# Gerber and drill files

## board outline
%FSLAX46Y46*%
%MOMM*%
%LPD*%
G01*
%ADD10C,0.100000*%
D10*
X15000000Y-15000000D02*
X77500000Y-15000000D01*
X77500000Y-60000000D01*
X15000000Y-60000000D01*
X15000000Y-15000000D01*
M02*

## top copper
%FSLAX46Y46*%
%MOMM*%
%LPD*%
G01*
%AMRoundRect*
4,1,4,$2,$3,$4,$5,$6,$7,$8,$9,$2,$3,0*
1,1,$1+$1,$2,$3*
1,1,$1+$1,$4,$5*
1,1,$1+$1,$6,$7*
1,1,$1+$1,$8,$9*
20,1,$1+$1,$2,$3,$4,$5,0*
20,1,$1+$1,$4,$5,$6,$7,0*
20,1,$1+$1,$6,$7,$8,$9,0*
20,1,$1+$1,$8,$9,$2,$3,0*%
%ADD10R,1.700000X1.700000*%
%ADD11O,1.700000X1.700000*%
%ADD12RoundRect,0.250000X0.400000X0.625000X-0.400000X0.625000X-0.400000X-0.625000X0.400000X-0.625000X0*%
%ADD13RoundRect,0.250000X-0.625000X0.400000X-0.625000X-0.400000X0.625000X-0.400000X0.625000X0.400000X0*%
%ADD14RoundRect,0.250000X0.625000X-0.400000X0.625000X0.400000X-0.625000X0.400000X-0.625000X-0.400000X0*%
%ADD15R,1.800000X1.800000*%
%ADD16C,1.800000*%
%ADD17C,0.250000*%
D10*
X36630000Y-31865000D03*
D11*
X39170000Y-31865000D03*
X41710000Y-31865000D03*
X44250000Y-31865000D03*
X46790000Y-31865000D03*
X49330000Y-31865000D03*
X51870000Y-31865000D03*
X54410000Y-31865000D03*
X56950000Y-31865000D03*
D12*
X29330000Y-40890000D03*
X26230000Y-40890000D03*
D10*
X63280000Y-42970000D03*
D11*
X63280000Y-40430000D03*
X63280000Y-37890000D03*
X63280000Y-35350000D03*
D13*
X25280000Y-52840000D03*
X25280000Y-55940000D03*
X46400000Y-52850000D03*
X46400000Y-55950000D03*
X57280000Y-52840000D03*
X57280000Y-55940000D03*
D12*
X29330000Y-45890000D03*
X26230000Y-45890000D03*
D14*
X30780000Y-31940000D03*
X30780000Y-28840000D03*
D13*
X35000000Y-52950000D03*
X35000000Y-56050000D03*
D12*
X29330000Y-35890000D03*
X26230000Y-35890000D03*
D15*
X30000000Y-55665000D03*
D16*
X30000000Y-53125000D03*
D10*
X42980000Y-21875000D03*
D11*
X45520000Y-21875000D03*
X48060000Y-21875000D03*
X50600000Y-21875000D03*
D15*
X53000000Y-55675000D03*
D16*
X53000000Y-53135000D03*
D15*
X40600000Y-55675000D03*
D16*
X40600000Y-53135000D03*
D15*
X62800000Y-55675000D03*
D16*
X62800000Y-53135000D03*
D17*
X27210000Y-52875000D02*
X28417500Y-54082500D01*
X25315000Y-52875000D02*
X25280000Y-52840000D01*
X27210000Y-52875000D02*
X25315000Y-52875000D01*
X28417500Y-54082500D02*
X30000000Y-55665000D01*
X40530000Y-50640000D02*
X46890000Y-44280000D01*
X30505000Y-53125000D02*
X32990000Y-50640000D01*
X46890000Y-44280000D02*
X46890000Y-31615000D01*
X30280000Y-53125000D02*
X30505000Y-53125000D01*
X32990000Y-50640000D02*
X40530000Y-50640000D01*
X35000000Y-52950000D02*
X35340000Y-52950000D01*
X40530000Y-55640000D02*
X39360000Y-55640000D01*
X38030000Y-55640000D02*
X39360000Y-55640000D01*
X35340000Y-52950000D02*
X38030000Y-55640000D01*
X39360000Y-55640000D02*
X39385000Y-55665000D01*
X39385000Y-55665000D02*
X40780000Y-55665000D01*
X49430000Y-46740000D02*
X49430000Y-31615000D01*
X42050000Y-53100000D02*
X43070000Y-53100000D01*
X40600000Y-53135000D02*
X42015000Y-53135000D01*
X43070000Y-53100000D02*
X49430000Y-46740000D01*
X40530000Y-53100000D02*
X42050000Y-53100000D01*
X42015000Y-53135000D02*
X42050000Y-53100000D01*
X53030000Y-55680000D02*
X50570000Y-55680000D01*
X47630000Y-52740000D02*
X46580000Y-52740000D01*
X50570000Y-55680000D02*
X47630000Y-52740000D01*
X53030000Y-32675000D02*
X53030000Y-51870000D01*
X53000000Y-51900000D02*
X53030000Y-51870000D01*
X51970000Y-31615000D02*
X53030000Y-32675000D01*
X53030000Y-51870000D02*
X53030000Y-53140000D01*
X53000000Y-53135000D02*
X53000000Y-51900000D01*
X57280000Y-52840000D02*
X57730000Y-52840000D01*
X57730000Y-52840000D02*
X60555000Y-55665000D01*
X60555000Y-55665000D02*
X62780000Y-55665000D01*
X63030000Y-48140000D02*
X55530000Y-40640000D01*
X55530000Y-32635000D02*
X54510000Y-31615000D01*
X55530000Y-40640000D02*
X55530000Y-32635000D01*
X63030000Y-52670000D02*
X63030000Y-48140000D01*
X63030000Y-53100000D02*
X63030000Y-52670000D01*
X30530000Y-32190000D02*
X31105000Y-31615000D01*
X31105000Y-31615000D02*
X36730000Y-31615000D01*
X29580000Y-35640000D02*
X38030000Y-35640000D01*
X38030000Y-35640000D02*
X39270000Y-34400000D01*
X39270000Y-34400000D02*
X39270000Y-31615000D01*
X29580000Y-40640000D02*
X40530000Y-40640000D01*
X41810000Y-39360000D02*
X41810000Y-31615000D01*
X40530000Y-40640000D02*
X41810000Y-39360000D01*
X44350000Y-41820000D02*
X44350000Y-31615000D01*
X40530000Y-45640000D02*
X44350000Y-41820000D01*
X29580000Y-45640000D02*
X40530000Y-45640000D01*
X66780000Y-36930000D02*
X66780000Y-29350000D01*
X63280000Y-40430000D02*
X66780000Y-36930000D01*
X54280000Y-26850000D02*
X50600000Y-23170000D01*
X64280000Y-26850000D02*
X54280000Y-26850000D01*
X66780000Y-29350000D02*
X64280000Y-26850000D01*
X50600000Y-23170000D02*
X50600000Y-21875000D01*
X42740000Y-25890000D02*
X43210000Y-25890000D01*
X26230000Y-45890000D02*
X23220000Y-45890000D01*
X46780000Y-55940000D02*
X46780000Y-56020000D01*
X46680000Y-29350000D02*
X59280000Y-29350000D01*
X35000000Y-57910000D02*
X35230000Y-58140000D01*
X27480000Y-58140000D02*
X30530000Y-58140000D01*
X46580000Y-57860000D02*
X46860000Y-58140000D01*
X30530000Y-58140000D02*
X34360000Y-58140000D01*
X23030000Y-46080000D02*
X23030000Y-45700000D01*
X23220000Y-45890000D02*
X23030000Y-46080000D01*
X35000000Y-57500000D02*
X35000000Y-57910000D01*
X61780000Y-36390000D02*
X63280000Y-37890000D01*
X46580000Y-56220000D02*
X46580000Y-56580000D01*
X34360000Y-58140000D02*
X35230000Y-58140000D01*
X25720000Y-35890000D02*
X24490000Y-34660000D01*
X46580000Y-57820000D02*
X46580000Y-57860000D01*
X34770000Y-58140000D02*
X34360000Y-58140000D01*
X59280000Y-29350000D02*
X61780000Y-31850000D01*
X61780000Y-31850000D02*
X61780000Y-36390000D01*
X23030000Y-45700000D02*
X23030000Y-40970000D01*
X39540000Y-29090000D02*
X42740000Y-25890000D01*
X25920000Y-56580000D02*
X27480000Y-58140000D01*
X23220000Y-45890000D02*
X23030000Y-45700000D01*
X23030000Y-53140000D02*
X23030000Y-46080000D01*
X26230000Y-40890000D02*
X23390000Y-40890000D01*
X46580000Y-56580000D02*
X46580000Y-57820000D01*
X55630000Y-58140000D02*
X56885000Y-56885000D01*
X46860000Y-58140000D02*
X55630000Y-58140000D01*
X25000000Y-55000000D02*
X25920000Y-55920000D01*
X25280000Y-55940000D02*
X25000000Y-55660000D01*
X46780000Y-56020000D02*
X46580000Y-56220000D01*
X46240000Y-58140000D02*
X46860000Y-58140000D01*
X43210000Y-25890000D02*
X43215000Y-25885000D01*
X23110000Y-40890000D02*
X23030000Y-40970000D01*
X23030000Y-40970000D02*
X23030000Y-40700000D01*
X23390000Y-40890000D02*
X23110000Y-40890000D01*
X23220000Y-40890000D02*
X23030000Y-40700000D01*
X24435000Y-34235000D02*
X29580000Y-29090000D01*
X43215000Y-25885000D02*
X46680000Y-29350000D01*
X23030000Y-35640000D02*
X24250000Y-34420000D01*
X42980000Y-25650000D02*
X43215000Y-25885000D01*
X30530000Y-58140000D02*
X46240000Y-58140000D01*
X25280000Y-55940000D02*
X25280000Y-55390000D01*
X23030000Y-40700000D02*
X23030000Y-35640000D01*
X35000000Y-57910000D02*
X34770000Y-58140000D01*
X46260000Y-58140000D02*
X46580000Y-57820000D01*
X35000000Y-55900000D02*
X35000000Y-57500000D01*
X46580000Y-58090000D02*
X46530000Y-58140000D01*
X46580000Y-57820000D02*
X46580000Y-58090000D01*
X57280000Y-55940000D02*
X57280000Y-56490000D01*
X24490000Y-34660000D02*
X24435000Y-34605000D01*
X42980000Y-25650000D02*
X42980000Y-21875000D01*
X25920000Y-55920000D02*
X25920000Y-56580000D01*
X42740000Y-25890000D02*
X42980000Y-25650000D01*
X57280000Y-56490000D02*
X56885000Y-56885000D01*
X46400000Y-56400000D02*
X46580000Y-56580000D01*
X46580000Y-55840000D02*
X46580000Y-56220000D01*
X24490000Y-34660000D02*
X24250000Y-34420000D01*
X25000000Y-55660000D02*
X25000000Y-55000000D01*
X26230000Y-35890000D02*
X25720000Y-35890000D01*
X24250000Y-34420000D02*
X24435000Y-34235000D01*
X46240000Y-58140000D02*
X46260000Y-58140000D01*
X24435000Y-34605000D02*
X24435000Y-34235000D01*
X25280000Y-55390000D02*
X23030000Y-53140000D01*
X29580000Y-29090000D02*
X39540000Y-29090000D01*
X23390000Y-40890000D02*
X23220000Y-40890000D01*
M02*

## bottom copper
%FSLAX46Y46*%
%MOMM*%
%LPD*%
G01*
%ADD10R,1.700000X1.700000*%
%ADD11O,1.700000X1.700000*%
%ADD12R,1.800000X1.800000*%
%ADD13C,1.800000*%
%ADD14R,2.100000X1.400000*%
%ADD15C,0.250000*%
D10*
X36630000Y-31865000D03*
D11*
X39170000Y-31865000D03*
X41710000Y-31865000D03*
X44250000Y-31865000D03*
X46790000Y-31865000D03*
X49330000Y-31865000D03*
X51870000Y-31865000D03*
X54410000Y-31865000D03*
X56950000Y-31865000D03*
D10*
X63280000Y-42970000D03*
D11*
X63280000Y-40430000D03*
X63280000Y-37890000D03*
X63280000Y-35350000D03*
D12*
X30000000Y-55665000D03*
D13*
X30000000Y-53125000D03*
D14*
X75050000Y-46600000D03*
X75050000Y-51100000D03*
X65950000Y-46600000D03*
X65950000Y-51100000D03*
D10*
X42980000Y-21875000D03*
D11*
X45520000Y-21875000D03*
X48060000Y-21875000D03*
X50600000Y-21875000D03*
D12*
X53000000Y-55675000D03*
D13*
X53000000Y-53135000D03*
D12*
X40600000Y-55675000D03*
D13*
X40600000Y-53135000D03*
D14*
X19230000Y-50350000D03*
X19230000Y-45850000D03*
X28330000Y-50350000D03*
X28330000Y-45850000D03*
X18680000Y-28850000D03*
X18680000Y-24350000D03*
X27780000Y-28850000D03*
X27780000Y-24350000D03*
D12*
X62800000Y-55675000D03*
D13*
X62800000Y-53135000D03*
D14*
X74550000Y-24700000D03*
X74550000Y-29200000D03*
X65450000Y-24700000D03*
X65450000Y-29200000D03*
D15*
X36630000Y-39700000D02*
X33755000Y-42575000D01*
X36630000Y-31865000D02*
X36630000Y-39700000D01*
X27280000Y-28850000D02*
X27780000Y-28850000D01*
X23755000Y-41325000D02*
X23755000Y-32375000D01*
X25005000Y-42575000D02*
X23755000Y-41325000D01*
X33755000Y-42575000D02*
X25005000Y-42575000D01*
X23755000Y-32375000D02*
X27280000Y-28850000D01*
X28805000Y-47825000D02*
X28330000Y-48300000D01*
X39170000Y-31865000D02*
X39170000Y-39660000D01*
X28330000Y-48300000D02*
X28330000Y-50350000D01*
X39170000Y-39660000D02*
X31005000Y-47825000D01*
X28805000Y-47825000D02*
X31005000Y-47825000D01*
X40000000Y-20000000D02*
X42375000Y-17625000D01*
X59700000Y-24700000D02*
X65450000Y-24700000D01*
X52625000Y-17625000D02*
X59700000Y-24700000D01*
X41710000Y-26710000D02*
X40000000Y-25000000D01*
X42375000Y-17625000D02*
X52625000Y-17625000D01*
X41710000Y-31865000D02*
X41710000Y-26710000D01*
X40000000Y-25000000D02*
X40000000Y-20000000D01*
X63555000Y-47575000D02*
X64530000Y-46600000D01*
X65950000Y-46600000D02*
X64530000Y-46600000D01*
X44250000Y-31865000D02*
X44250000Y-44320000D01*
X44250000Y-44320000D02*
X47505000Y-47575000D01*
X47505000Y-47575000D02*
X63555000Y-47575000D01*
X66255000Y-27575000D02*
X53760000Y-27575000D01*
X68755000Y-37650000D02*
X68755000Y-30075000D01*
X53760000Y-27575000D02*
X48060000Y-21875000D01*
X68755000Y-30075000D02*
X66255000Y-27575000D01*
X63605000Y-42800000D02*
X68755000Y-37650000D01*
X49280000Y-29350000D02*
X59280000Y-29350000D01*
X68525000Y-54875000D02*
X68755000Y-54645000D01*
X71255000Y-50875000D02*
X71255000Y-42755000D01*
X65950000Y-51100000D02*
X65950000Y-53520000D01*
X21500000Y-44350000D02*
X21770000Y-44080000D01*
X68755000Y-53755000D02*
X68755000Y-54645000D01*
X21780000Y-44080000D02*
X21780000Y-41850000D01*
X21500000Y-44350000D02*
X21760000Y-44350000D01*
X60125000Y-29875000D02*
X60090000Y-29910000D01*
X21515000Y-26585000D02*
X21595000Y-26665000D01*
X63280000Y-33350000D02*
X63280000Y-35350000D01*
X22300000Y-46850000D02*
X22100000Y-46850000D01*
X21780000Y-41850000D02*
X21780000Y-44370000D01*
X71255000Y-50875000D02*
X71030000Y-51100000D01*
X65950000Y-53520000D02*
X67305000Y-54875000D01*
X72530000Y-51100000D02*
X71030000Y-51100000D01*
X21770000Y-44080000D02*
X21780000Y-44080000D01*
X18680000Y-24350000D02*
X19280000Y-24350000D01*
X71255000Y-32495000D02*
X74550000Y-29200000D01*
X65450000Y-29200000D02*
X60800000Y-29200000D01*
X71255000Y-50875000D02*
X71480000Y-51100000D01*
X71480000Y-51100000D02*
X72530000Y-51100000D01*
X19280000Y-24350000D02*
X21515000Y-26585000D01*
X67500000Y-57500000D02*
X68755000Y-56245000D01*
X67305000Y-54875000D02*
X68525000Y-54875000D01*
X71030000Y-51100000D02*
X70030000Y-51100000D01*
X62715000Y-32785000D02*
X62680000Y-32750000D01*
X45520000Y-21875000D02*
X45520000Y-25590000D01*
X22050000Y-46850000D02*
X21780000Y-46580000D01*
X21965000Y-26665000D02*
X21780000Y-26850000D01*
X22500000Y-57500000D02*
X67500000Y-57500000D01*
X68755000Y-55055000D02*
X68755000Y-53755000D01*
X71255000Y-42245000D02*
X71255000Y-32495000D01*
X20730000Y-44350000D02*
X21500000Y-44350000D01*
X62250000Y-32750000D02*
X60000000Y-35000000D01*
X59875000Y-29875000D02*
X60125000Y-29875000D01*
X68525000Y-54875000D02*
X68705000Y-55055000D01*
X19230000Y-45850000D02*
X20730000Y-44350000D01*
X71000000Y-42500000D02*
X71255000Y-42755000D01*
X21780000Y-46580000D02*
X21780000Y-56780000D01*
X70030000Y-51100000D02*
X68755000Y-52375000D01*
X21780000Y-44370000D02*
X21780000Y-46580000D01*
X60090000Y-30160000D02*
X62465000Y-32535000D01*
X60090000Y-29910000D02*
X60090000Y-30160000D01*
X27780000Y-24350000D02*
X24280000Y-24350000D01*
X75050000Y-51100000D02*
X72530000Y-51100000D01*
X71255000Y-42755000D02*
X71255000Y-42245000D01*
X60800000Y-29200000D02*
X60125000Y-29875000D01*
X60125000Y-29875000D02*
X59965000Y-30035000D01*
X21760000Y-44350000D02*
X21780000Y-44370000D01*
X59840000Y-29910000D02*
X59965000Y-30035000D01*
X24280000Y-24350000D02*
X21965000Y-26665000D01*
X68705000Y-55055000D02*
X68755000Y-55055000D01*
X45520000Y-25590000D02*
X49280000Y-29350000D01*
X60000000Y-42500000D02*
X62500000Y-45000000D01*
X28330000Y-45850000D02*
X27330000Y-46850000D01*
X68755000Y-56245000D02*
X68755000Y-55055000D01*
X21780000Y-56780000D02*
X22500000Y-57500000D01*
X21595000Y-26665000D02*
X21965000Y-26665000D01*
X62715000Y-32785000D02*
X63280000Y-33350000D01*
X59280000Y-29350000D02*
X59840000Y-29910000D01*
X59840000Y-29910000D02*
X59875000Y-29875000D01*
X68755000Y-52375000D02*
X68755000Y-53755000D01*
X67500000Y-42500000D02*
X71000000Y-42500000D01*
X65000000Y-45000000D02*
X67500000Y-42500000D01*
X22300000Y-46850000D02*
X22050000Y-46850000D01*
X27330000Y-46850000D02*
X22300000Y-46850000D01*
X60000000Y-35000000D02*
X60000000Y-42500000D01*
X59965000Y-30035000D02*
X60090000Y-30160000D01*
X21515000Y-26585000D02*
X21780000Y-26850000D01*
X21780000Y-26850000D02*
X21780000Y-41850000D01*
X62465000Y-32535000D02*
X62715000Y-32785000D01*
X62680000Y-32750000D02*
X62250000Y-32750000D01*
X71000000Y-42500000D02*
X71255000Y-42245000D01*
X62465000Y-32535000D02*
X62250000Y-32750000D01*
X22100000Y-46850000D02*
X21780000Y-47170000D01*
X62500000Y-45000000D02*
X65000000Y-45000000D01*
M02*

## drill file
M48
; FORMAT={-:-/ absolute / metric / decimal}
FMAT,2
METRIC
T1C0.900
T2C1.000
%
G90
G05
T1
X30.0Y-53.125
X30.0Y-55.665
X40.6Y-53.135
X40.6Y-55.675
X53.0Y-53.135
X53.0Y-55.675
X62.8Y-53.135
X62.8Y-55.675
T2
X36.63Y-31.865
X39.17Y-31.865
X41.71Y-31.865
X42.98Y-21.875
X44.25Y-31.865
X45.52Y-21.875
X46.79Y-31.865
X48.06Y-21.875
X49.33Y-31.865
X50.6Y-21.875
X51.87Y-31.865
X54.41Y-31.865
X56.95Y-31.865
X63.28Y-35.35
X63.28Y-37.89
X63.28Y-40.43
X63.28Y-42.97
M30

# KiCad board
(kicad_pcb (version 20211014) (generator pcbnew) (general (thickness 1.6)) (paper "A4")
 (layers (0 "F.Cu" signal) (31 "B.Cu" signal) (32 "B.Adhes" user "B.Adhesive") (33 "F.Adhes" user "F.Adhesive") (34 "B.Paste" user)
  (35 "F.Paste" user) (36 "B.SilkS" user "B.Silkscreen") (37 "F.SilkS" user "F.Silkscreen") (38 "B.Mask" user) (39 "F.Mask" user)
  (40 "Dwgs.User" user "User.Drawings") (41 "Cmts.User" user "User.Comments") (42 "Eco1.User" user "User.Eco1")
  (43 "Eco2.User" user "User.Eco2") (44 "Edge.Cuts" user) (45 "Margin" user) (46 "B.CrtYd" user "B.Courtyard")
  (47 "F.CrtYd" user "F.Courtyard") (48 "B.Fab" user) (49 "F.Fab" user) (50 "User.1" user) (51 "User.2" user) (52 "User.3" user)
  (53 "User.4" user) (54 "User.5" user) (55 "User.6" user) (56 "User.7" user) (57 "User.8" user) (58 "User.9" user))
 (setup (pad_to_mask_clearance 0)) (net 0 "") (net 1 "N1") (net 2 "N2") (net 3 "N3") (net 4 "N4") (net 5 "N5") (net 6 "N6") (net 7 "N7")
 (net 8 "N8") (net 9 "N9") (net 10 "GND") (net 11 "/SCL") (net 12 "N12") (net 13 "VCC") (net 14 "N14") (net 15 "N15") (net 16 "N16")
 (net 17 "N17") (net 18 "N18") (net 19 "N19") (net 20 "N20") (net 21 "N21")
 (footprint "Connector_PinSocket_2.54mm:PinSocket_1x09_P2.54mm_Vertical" (layer "F.Cu") (at 36.63 31.865 90)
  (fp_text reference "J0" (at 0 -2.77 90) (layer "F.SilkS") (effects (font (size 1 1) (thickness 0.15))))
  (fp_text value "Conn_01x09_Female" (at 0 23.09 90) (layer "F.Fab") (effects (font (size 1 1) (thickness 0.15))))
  (pad "1" thru_hole rect (at 0 0 90) (size 1.7 1.7) (drill 1) (layers *.Cu *.Mask) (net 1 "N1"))
  (pad "2" thru_hole oval (at 0 2.54 90) (size 1.7 1.7) (drill 1) (layers *.Cu *.Mask) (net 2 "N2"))
  (pad "3" thru_hole oval (at 0 5.08 90) (size 1.7 1.7) (drill 1) (layers *.Cu *.Mask) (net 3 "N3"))
  (pad "4" thru_hole oval (at 0 7.62 90) (size 1.7 1.7) (drill 1) (layers *.Cu *.Mask) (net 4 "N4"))
  (pad "5" thru_hole oval (at 0 10.16 90) (size 1.7 1.7) (drill 1) (layers *.Cu *.Mask) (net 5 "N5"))
  (pad "6" thru_hole oval (at 0 12.7 90) (size 1.7 1.7) (drill 1) (layers *.Cu *.Mask) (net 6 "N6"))
  (pad "7" thru_hole oval (at 0 15.24 90) (size 1.7 1.7) (drill 1) (layers *.Cu *.Mask) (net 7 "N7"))
  (pad "8" thru_hole oval (at 0 17.78 90) (size 1.7 1.7) (drill 1) (layers *.Cu *.Mask) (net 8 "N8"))
  (pad "9" thru_hole oval (at 0 20.32 90) (size 1.7 1.7) (drill 1) (layers *.Cu *.Mask) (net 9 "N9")))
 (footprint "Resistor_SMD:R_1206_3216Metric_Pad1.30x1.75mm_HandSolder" (layer "F.Cu") (at 27.78 40.89 180)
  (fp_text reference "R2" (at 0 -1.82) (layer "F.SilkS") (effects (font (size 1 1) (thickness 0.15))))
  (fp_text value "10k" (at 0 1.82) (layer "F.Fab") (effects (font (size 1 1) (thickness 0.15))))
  (pad "1" smd roundrect (at -1.55 0 180) (size 1.3 1.75) (layers "F.Cu" "F.Paste" "F.Mask") (roundrect_rratio 0.192308) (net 3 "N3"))
  (pad "2" smd roundrect (at 1.55 0 180) (size 1.3 1.75) (layers "F.Cu" "F.Paste" "F.Mask") (roundrect_rratio 0.192308) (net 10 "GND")))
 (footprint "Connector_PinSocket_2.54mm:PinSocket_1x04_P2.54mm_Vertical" (layer "F.Cu") (at 63.28 42.97 180)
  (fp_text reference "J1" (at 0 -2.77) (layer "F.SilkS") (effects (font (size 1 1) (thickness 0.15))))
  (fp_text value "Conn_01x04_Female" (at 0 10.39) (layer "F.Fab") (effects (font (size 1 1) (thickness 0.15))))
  (pad "1" thru_hole rect (at 0 0 180) (size 1.7 1.7) (drill 1) (layers *.Cu *.Mask) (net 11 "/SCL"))
  (pad "2" thru_hole oval (at 0 2.54 180) (size 1.7 1.7) (drill 1) (layers *.Cu *.Mask) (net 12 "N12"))
  (pad "3" thru_hole oval (at 0 5.08 180) (size 1.7 1.7) (drill 1) (layers *.Cu *.Mask) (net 10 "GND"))
  (pad "4" thru_hole oval (at 0 7.62 180) (size 1.7 1.7) (drill 1) (layers *.Cu *.Mask) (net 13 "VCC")))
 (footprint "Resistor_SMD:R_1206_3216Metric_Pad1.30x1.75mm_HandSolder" (layer "F.Cu") (at 25.28 54.39 -90)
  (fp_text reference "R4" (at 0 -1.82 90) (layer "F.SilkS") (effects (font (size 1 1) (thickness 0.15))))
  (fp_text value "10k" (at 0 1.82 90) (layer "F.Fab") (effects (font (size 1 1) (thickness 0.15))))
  (pad "1" smd roundrect (at -1.55 0 270) (size 1.3 1.75) (layers "F.Cu" "F.Paste" "F.Mask") (roundrect_rratio 0.192308) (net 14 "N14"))
  (pad "2" smd roundrect (at 1.55 0 270) (size 1.3 1.75) (layers "F.Cu" "F.Paste" "F.Mask") (roundrect_rratio 0.192308) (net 10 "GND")))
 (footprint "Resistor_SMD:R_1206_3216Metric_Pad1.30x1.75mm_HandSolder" (layer "F.Cu") (at 46.4 54.4 -90)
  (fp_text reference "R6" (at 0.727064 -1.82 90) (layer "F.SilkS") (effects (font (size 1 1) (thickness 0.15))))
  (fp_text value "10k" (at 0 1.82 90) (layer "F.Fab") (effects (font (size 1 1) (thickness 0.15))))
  (pad "1" smd roundrect (at -1.55 0 270) (size 1.3 1.75) (layers "F.Cu" "F.Paste" "F.Mask") (roundrect_rratio 0.192308) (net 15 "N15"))
  (pad "2" smd roundrect (at 1.55 0 270) (size 1.3 1.75) (layers "F.Cu" "F.Paste" "F.Mask") (roundrect_rratio 0.192308) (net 10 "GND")))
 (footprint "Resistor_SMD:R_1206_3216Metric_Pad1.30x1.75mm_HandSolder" (layer "F.Cu") (at 57.28 54.39 -90)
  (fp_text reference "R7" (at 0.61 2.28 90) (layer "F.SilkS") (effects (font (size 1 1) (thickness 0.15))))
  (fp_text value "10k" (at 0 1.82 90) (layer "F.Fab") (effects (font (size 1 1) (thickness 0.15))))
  (pad "1" smd roundrect (at -1.55 0 270) (size 1.3 1.75) (layers "F.Cu" "F.Paste" "F.Mask") (roundrect_rratio 0.192308) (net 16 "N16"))
  (pad "2" smd roundrect (at 1.55 0 270) (size 1.3 1.75) (layers "F.Cu" "F.Paste" "F.Mask") (roundrect_rratio 0.192308) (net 10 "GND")))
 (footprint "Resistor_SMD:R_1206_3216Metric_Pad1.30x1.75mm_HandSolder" (layer "F.Cu") (at 27.78 45.89 180)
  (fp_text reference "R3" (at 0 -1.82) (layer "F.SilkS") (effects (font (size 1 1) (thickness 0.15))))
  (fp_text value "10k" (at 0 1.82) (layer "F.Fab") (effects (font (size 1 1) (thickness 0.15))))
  (pad "1" smd roundrect (at -1.55 0 180) (size 1.3 1.75) (layers "F.Cu" "F.Paste" "F.Mask") (roundrect_rratio 0.192308) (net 4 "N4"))
  (pad "2" smd roundrect (at 1.55 0 180) (size 1.3 1.75) (layers "F.Cu" "F.Paste" "F.Mask") (roundrect_rratio 0.192308) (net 10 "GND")))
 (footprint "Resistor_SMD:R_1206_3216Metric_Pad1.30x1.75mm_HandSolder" (layer "F.Cu") (at 30.78 30.39 90)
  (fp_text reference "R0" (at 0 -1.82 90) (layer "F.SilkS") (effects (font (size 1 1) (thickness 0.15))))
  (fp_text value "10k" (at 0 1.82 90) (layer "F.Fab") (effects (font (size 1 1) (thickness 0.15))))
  (pad "1" smd roundrect (at -1.55 0 90) (size 1.3 1.75) (layers "F.Cu" "F.Paste" "F.Mask") (roundrect_rratio 0.192308) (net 1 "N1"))
  (pad "2" smd roundrect (at 1.55 0 90) (size 1.3 1.75) (layers "F.Cu" "F.Paste" "F.Mask") (roundrect_rratio 0.192308) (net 10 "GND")))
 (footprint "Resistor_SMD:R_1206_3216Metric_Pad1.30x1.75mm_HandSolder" (layer "F.Cu") (at 35 54.5 -90)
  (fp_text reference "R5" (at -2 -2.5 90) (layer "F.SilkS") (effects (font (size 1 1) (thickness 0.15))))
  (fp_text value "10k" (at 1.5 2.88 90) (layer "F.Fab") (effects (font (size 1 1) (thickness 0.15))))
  (pad "1" smd roundrect (at -1.55 0 270) (size 1.3 1.75) (layers "F.Cu" "F.Paste" "F.Mask") (roundrect_rratio 0.192308) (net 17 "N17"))
  (pad "2" smd roundrect (at 1.55 0 270) (size 1.3 1.75) (layers "F.Cu" "F.Paste" "F.Mask") (roundrect_rratio 0.192308) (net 10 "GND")))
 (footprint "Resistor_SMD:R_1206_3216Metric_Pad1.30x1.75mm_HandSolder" (layer "F.Cu") (at 27.78 35.89 180)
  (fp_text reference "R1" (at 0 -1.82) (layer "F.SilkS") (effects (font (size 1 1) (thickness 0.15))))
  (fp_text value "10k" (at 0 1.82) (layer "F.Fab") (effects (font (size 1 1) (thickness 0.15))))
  (pad "1" smd roundrect (at -1.55 0 180) (size 1.3 1.75) (layers "F.Cu" "F.Paste" "F.Mask") (roundrect_rratio 0.192308) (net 2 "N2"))
  (pad "2" smd roundrect (at 1.55 0 180) (size 1.3 1.75) (layers "F.Cu" "F.Paste" "F.Mask") (roundrect_rratio 0.192308) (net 10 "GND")))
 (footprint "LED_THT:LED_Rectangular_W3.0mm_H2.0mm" (layer "B.Cu") (at 30 55.665 90)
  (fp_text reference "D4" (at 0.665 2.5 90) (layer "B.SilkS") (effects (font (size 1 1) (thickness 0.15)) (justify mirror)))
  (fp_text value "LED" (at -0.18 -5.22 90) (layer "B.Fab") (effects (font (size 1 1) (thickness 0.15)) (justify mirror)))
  (pad "1" thru_hole rect (at 0 0 90) (size 1.8 1.8) (drill 0.9) (layers *.Cu *.Mask) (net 14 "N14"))
  (pad "2" thru_hole circle (at 2.54 0 90) (size 1.8 1.8) (drill 0.9) (layers *.Cu *.Mask) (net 5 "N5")))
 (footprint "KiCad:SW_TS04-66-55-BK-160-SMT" (layer "B.Cu") (at 70.5 48.85 180)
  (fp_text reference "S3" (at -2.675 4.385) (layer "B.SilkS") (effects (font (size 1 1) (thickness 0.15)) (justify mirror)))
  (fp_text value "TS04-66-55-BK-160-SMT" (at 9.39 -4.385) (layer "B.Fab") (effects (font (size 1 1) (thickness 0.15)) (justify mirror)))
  (pad "1" smd rect locked (at -4.55 2.25 180) (size 2.1 1.4) (layers "B.Cu" "B.Paste" "B.Mask") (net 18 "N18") (solder_mask_margin 0.102))
  (pad "2" smd rect locked (at -4.55 -2.25 180) (size 2.1 1.4) (layers "B.Cu" "B.Paste" "B.Mask") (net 13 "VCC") (solder_mask_margin 0.102))
  (pad "3" smd rect locked (at 4.55 2.25 180) (size 2.1 1.4) (layers "B.Cu" "B.Paste" "B.Mask") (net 4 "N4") (solder_mask_margin 0.102))
  (pad "4" smd rect locked (at 4.55 -2.25 180) (size 2.1 1.4) (layers "B.Cu" "B.Paste" "B.Mask") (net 13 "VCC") (solder_mask_margin 0.102)))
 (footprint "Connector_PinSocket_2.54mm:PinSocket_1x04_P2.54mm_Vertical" (layer "B.Cu") (at 42.98 21.875 -90)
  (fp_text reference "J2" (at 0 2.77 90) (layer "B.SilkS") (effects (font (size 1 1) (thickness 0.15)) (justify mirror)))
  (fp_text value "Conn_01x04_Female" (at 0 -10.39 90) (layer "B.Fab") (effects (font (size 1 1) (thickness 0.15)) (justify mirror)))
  (pad "1" thru_hole rect (at 0 0 270) (size 1.7 1.7) (drill 1) (layers *.Cu *.Mask) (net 10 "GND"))
  (pad "2" thru_hole oval (at 0 -2.54 270) (size 1.7 1.7) (drill 1) (layers *.Cu *.Mask) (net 13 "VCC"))
  (pad "3" thru_hole oval (at 0 -5.08 270) (size 1.7 1.7) (drill 1) (layers *.Cu *.Mask) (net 11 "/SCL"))
  (pad "4" thru_hole oval (at 0 -7.62 270) (size 1.7 1.7) (drill 1) (layers *.Cu *.Mask) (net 12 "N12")))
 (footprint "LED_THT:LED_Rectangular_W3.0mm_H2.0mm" (layer "B.Cu") (at 53 55.675 90)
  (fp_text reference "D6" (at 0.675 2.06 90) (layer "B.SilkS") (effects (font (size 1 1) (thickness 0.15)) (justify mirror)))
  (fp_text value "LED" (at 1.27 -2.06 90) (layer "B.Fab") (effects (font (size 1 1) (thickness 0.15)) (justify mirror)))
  (pad "1" thru_hole rect (at 0 0 90) (size 1.8 1.8) (drill 0.9) (layers *.Cu *.Mask) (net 15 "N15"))
  (pad "2" thru_hole circle (at 2.54 0 90) (size 1.8 1.8) (drill 0.9) (layers *.Cu *.Mask) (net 7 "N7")))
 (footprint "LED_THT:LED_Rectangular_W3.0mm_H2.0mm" (layer "B.Cu") (at 40.6 55.675 90)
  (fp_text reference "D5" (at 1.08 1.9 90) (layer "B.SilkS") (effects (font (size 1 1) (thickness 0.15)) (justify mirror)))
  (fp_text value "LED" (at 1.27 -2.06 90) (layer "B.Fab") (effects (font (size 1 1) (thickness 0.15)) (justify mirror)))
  (pad "1" thru_hole rect (at 0 0 90) (size 1.8 1.8) (drill 0.9) (layers *.Cu *.Mask) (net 17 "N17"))
  (pad "2" thru_hole circle (at 2.54 0 90) (size 1.8 1.8) (drill 0.9) (layers *.Cu *.Mask) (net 6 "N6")))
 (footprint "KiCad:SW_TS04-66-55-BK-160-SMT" (layer "B.Cu") (at 23.78 48.1)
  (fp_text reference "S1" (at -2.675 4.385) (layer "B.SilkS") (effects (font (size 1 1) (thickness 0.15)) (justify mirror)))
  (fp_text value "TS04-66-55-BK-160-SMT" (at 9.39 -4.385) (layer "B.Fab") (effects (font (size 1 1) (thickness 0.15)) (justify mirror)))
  (pad "1" smd rect locked (at -4.55 2.25) (size 2.1 1.4) (layers "B.Cu" "B.Paste" "B.Mask") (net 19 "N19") (solder_mask_margin 0.102))
  (pad "2" smd rect locked (at -4.55 -2.25) (size 2.1 1.4) (layers "B.Cu" "B.Paste" "B.Mask") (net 13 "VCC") (solder_mask_margin 0.102))
  (pad "3" smd rect locked (at 4.55 2.25) (size 2.1 1.4) (layers "B.Cu" "B.Paste" "B.Mask") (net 2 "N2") (solder_mask_margin 0.102))
  (pad "4" smd rect locked (at 4.55 -2.25) (size 2.1 1.4) (layers "B.Cu" "B.Paste" "B.Mask") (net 13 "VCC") (solder_mask_margin 0.102)))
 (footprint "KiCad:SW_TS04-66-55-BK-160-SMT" (layer "B.Cu") (at 23.23 26.6)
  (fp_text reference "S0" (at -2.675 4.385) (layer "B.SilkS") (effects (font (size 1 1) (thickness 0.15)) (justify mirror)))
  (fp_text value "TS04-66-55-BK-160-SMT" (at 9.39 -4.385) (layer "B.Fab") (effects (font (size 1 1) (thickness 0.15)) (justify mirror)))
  (pad "1" smd rect locked (at -4.55 2.25) (size 2.1 1.4) (layers "B.Cu" "B.Paste" "B.Mask") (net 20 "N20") (solder_mask_margin 0.102))
  (pad "2" smd rect locked (at -4.55 -2.25) (size 2.1 1.4) (layers "B.Cu" "B.Paste" "B.Mask") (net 13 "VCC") (solder_mask_margin 0.102))
  (pad "3" smd rect locked (at 4.55 2.25) (size 2.1 1.4) (layers "B.Cu" "B.Paste" "B.Mask") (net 1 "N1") (solder_mask_margin 0.102))
  (pad "4" smd rect locked (at 4.55 -2.25) (size 2.1 1.4) (layers "B.Cu" "B.Paste" "B.Mask") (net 13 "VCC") (solder_mask_margin 0.102)))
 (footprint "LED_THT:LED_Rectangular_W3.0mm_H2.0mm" (layer "B.Cu") (at 62.8 55.675 90)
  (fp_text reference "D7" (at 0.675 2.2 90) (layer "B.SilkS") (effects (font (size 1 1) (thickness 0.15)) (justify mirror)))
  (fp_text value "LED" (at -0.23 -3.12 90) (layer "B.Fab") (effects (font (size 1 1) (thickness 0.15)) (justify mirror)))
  (pad "1" thru_hole rect (at 0 0 90) (size 1.8 1.8) (drill 0.9) (layers *.Cu *.Mask) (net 16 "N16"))
  (pad "2" thru_hole circle (at 2.54 0 90) (size 1.8 1.8) (drill 0.9) (layers *.Cu *.Mask) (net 8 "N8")))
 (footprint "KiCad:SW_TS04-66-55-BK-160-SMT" (layer "B.Cu") (at 70 26.95 180)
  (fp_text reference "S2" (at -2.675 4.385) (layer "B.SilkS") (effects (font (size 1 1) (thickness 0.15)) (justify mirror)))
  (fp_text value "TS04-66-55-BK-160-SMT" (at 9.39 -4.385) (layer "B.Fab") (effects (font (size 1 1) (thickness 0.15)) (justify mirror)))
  (pad "1" smd rect locked (at -4.55 2.25 180) (size 2.1 1.4) (layers "B.Cu" "B.Paste" "B.Mask") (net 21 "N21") (solder_mask_margin 0.102))
  (pad "2" smd rect locked (at -4.55 -2.25 180) (size 2.1 1.4) (layers "B.Cu" "B.Paste" "B.Mask") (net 13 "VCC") (solder_mask_margin 0.102))
  (pad "3" smd rect locked (at 4.55 2.25 180) (size 2.1 1.4) (layers "B.Cu" "B.Paste" "B.Mask") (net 3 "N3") (solder_mask_margin 0.102))
  (pad "4" smd rect locked (at 4.55 -2.25 180) (size 2.1 1.4) (layers "B.Cu" "B.Paste" "B.Mask") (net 13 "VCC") (solder_mask_margin 0.102)))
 (gr_rect (start 15 15) (end 77.5 60) (layer "Edge.Cuts") (width 0.1) (fill none))
 (gr_rect (start 12.5 15) (end 12.5 15) (layer "Edge.Cuts") (width 0.1) (fill none))
 (segment (start 27.21 52.875) (end 28.4175 54.0825) (width 0.25) (layer "F.Cu") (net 14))
 (segment (start 25.315 52.875) (end 25.28 52.84) (width 0.25) (layer "F.Cu") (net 14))
 (segment (start 27.21 52.875) (end 25.315 52.875) (width 0.25) (layer "F.Cu") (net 14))
 (segment (start 28.4175 54.0825) (end 30 55.665) (width 0.25) (layer "F.Cu") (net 14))
 (segment (start 40.53 50.64) (end 46.89 44.28) (width 0.25) (layer "F.Cu") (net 5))
 (segment (start 30.505 53.125) (end 32.99 50.64) (width 0.25) (layer "F.Cu") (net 5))
 (segment (start 46.89 44.28) (end 46.89 31.615) (width 0.25) (layer "F.Cu") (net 5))
 (segment (start 30.28 53.125) (end 30.505 53.125) (width 0.25) (layer "F.Cu") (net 5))
 (segment (start 32.99 50.64) (end 40.53 50.64) (width 0.25) (layer "F.Cu") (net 5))
 (segment (start 35 52.95) (end 35.34 52.95) (width 0.25) (layer "F.Cu") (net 17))
 (segment (start 40.53 55.64) (end 39.36 55.64) (width 0.25) (layer "F.Cu") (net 17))
 (segment (start 38.03 55.64) (end 39.36 55.64) (width 0.25) (layer "F.Cu") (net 17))
 (segment (start 35.34 52.95) (end 38.03 55.64) (width 0.25) (layer "F.Cu") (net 17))
 (segment (start 39.36 55.64) (end 39.385 55.665) (width 0.25) (layer "F.Cu") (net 17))
 (segment (start 39.385 55.665) (end 40.78 55.665) (width 0.25) (layer "F.Cu") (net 17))
 (segment (start 49.43 46.74) (end 49.43 31.615) (width 0.25) (layer "F.Cu") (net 6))
 (segment (start 42.05 53.1) (end 43.07 53.1) (width 0.25) (layer "F.Cu") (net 6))
 (segment (start 40.6 53.135) (end 42.015 53.135) (width 0.25) (layer "F.Cu") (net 6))
 (segment (start 43.07 53.1) (end 49.43 46.74) (width 0.25) (layer "F.Cu") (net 6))
 (segment (start 40.53 53.1) (end 42.05 53.1) (width 0.25) (layer "F.Cu") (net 6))
 (segment (start 42.015 53.135) (end 42.05 53.1) (width 0.25) (layer "F.Cu") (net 6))
 (segment (start 53.03 55.68) (end 50.57 55.68) (width 0.25) (layer "F.Cu") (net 15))
 (segment (start 47.63 52.74) (end 46.58 52.74) (width 0.25) (layer "F.Cu") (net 15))
 (segment (start 50.57 55.68) (end 47.63 52.74) (width 0.25) (layer "F.Cu") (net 15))
 (segment (start 53.03 32.675) (end 53.03 51.87) (width 0.25) (layer "F.Cu") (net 7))
 (segment (start 53 51.9) (end 53.03 51.87) (width 0.25) (layer "F.Cu") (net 7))
 (segment (start 51.97 31.615) (end 53.03 32.675) (width 0.25) (layer "F.Cu") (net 7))
 (segment (start 53.03 51.87) (end 53.03 53.14) (width 0.25) (layer "F.Cu") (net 7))
 (segment (start 53 53.135) (end 53 51.9) (width 0.25) (layer "F.Cu") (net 7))
 (segment (start 57.28 52.84) (end 57.73 52.84) (width 0.25) (layer "F.Cu") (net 16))
 (segment (start 57.73 52.84) (end 60.555 55.665) (width 0.25) (layer "F.Cu") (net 16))
 (segment (start 60.555 55.665) (end 62.78 55.665) (width 0.25) (layer "F.Cu") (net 16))
 (segment (start 63.03 48.14) (end 55.53 40.64) (width 0.25) (layer "F.Cu") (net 8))
 (segment (start 55.53 32.635) (end 54.51 31.615) (width 0.25) (layer "F.Cu") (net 8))
 (segment (start 55.53 40.64) (end 55.53 32.635) (width 0.25) (layer "F.Cu") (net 8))
 (segment (start 63.03 52.67) (end 63.03 48.14) (width 0.25) (layer "F.Cu") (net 8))
 (segment (start 63.03 53.1) (end 63.03 52.67) (width 0.25) (layer "F.Cu") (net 8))
 (segment (start 30.53 32.19) (end 31.105 31.615) (width 0.25) (layer "F.Cu") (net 1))
 (segment (start 31.105 31.615) (end 36.73 31.615) (width 0.25) (layer "F.Cu") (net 1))
 (segment (start 36.63 39.7) (end 33.755 42.575) (width 0.25) (layer "B.Cu") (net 1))
 (segment (start 36.63 31.865) (end 36.63 39.7) (width 0.25) (layer "B.Cu") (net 1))
 (segment (start 27.28 28.85) (end 27.78 28.85) (width 0.25) (layer "B.Cu") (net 1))
 (segment (start 23.755 41.325) (end 23.755 32.375) (width 0.25) (layer "B.Cu") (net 1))
 (segment (start 25.005 42.575) (end 23.755 41.325) (width 0.25) (layer "B.Cu") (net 1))
 (segment (start 33.755 42.575) (end 25.005 42.575) (width 0.25) (layer "B.Cu") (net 1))
 (segment (start 23.755 32.375) (end 27.28 28.85) (width 0.25) (layer "B.Cu") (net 1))
 (segment (start 29.58 35.64) (end 38.03 35.64) (width 0.25) (layer "F.Cu") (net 2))
 (segment (start 38.03 35.64) (end 39.27 34.4) (width 0.25) (layer "F.Cu") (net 2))
 (segment (start 39.27 34.4) (end 39.27 31.615) (width 0.25) (layer "F.Cu") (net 2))
 (segment (start 28.805 47.825) (end 28.33 48.3) (width 0.25) (layer "B.Cu") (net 2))
 (segment (start 39.17 31.865) (end 39.17 39.66) (width 0.25) (layer "B.Cu") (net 2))
 (segment (start 28.33 48.3) (end 28.33 50.35) (width 0.25) (layer "B.Cu") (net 2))
 (segment (start 39.17 39.66) (end 31.005 47.825) (width 0.25) (layer "B.Cu") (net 2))
 (segment (start 28.805 47.825) (end 31.005 47.825) (width 0.25) (layer "B.Cu") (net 2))
 (segment (start 29.58 40.64) (end 40.53 40.64) (width 0.25) (layer "F.Cu") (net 3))
 (segment (start 41.81 39.36) (end 41.81 31.615) (width 0.25) (layer "F.Cu") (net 3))
 (segment (start 40.53 40.64) (end 41.81 39.36) (width 0.25) (layer "F.Cu") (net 3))
 (segment (start 40 20) (end 42.375 17.625) (width 0.25) (layer "B.Cu") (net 3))
 (segment (start 59.7 24.7) (end 65.45 24.7) (width 0.25) (layer "B.Cu") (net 3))
 (segment (start 52.625 17.625) (end 59.7 24.7) (width 0.25) (layer "B.Cu") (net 3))
 (segment (start 41.71 26.71) (end 40 25) (width 0.25) (layer "B.Cu") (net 3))
 (segment (start 42.375 17.625) (end 52.625 17.625) (width 0.25) (layer "B.Cu") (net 3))
 (segment (start 41.71 31.865) (end 41.71 26.71) (width 0.25) (layer "B.Cu") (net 3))
 (segment (start 40 25) (end 40 20) (width 0.25) (layer "B.Cu") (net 3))
 (segment (start 44.35 41.82) (end 44.35 31.615) (width 0.25) (layer "F.Cu") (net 4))
 (segment (start 40.53 45.64) (end 44.35 41.82) (width 0.25) (layer "F.Cu") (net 4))
 (segment (start 29.58 45.64) (end 40.53 45.64) (width 0.25) (layer "F.Cu") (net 4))
 (segment (start 63.555 47.575) (end 64.53 46.6) (width 0.25) (layer "B.Cu") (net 4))
 (segment (start 65.95 46.6) (end 64.53 46.6) (width 0.25) (layer "B.Cu") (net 4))
 (segment (start 44.25 31.865) (end 44.25 44.32) (width 0.25) (layer "B.Cu") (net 4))
 (segment (start 44.25 44.32) (end 47.505 47.575) (width 0.25) (layer "B.Cu") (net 4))
 (segment (start 47.505 47.575) (end 63.555 47.575) (width 0.25) (layer "B.Cu") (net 4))
 (segment (start 66.255 27.575) (end 53.76 27.575) (width 0.25) (layer "B.Cu") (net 11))
 (segment (start 68.755 37.65) (end 68.755 30.075) (width 0.25) (layer "B.Cu") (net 11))
 (segment (start 53.76 27.575) (end 48.06 21.875) (width 0.25) (layer "B.Cu") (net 11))
 (segment (start 68.755 30.075) (end 66.255 27.575) (width 0.25) (layer "B.Cu") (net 11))
 (segment (start 63.605 42.8) (end 68.755 37.65) (width 0.25) (layer "B.Cu") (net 11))
 (segment (start 66.78 36.93) (end 66.78 29.35) (width 0.25) (layer "F.Cu") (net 12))
 (segment (start 63.28 40.43) (end 66.78 36.93) (width 0.25) (layer "F.Cu") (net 12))
 (segment (start 54.28 26.85) (end 50.6 23.17) (width 0.25) (layer "F.Cu") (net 12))
 (segment (start 64.28 26.85) (end 54.28 26.85) (width 0.25) (layer "F.Cu") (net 12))
 (segment (start 66.78 29.35) (end 64.28 26.85) (width 0.25) (layer "F.Cu") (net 12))
 (segment (start 50.6 23.17) (end 50.6 21.875) (width 0.25) (layer "F.Cu") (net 12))
 (segment (start 42.74 25.89) (end 43.21 25.89) (width 0.25) (layer "F.Cu") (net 10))
 (segment (start 26.23 45.89) (end 23.22 45.89) (width 0.25) (layer "F.Cu") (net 10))
 (segment (start 46.78 55.94) (end 46.78 56.02) (width 0.25) (layer "F.Cu") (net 10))
 (segment (start 46.68 29.35) (end 59.28 29.35) (width 0.25) (layer "F.Cu") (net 10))
 (segment (start 35 57.91) (end 35.23 58.14) (width 0.25) (layer "F.Cu") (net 10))
 (segment (start 27.48 58.14) (end 30.53 58.14) (width 0.25) (layer "F.Cu") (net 10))
 (segment (start 46.58 57.86) (end 46.86 58.14) (width 0.25) (layer "F.Cu") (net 10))
 (segment (start 30.53 58.14) (end 34.36 58.14) (width 0.25) (layer "F.Cu") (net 10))
 (segment (start 23.03 46.08) (end 23.03 45.7) (width 0.25) (layer "F.Cu") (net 10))
 (segment (start 23.22 45.89) (end 23.03 46.08) (width 0.25) (layer "F.Cu") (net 10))
 (segment (start 35 57.5) (end 35 57.91) (width 0.25) (layer "F.Cu") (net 10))
 (segment (start 61.78 36.39) (end 63.28 37.89) (width 0.25) (layer "F.Cu") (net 10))
 (segment (start 46.58 56.22) (end 46.58 56.58) (width 0.25) (layer "F.Cu") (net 10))
 (segment (start 34.36 58.14) (end 35.23 58.14) (width 0.25) (layer "F.Cu") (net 10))
 (segment (start 25.72 35.89) (end 24.49 34.66) (width 0.25) (layer "F.Cu") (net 10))
 (segment (start 46.58 57.82) (end 46.58 57.86) (width 0.25) (layer "F.Cu") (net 10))
 (segment (start 34.77 58.14) (end 34.36 58.14) (width 0.25) (layer "F.Cu") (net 10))
 (segment (start 59.28 29.35) (end 61.78 31.85) (width 0.25) (layer "F.Cu") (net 10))
 (segment (start 61.78 31.85) (end 61.78 36.39) (width 0.25) (layer "F.Cu") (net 10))
 (segment (start 23.03 45.7) (end 23.03 40.97) (width 0.25) (layer "F.Cu") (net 10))
 (segment (start 39.54 29.09) (end 42.74 25.89) (width 0.25) (layer "F.Cu") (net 10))
 (segment (start 25.92 56.58) (end 27.48 58.14) (width 0.25) (layer "F.Cu") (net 10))
 (segment (start 23.22 45.89) (end 23.03 45.7) (width 0.25) (layer "F.Cu") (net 10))
 (segment (start 23.03 53.14) (end 23.03 46.08) (width 0.25) (layer "F.Cu") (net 10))
 (segment (start 26.23 40.89) (end 23.39 40.89) (width 0.25) (layer "F.Cu") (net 10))
 (segment (start 46.58 56.58) (end 46.58 57.82) (width 0.25) (layer "F.Cu") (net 10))
 (segment (start 55.63 58.14) (end 56.885 56.885) (width 0.25) (layer "F.Cu") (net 10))
 (segment (start 46.86 58.14) (end 55.63 58.14) (width 0.25) (layer "F.Cu") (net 10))
 (segment (start 25 55) (end 25.92 55.92) (width 0.25) (layer "F.Cu") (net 10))
 (segment (start 25.28 55.94) (end 25 55.66) (width 0.25) (layer "F.Cu") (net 10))
 (segment (start 46.78 56.02) (end 46.58 56.22) (width 0.25) (layer "F.Cu") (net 10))
 (segment (start 46.24 58.14) (end 46.86 58.14) (width 0.25) (layer "F.Cu") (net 10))
 (segment (start 43.21 25.89) (end 43.215 25.885) (width 0.25) (layer "F.Cu") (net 10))
 (segment (start 23.11 40.89) (end 23.03 40.97) (width 0.25) (layer "F.Cu") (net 10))
 (segment (start 23.03 40.97) (end 23.03 40.7) (width 0.25) (layer "F.Cu") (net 10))
 (segment (start 23.39 40.89) (end 23.11 40.89) (width 0.25) (layer "F.Cu") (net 10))
 (segment (start 23.22 40.89) (end 23.03 40.7) (width 0.25) (layer "F.Cu") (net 10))
 (segment (start 24.435 34.235) (end 29.58 29.09) (width 0.25) (layer "F.Cu") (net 10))
 (segment (start 43.215 25.885) (end 46.68 29.35) (width 0.25) (layer "F.Cu") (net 10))
 (segment (start 23.03 35.64) (end 24.25 34.42) (width 0.25) (layer "F.Cu") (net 10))
 (segment (start 42.98 25.65) (end 43.215 25.885) (width 0.25) (layer "F.Cu") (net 10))
 (segment (start 30.53 58.14) (end 46.24 58.14) (width 0.25) (layer "F.Cu") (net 10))
 (segment (start 25.28 55.94) (end 25.28 55.39) (width 0.25) (layer "F.Cu") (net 10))
 (segment (start 23.03 40.7) (end 23.03 35.64) (width 0.25) (layer "F.Cu") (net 10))
 (segment (start 35 57.91) (end 34.77 58.14) (width 0.25) (layer "F.Cu") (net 10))
 (segment (start 46.26 58.14) (end 46.58 57.82) (width 0.25) (layer "F.Cu") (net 10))
 (segment (start 35 55.9) (end 35 57.5) (width 0.25) (layer "F.Cu") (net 10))
 (segment (start 46.58 58.09) (end 46.53 58.14) (width 0.25) (layer "F.Cu") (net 10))
 (segment (start 46.58 57.82) (end 46.58 58.09) (width 0.25) (layer "F.Cu") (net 10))
 (segment (start 57.28 55.94) (end 57.28 56.49) (width 0.25) (layer "F.Cu") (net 10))
 (segment (start 24.49 34.66) (end 24.435 34.605) (width 0.25) (layer "F.Cu") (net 10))
 (segment (start 42.98 25.65) (end 42.98 21.875) (width 0.25) (layer "F.Cu") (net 10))
 (segment (start 25.92 55.92) (end 25.92 56.58) (width 0.25) (layer "F.Cu") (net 10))
 (segment (start 42.74 25.89) (end 42.98 25.65) (width 0.25) (layer "F.Cu") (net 10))
 (segment (start 57.28 56.49) (end 56.885 56.885) (width 0.25) (layer "F.Cu") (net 10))
 (segment (start 46.4 56.4) (end 46.58 56.58) (width 0.25) (layer "F.Cu") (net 10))
 (segment (start 46.58 55.84) (end 46.58 56.22) (width 0.25) (layer "F.Cu") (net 10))
 (segment (start 24.49 34.66) (end 24.25 34.42) (width 0.25) (layer "F.Cu") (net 10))
 (segment (start 25 55.66) (end 25 55) (width 0.25) (layer "F.Cu") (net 10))
 (segment (start 26.23 35.89) (end 25.72 35.89) (width 0.25) (layer "F.Cu") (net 10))
 (segment (start 24.25 34.42) (end 24.435 34.235) (width 0.25) (layer "F.Cu") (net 10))
 (segment (start 46.24 58.14) (end 46.26 58.14) (width 0.25) (layer "F.Cu") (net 10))
 (segment (start 24.435 34.605) (end 24.435 34.235) (width 0.25) (layer "F.Cu") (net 10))
 (segment (start 25.28 55.39) (end 23.03 53.14) (width 0.25) (layer "F.Cu") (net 10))
 (segment (start 29.58 29.09) (end 39.54 29.09) (width 0.25) (layer "F.Cu") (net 10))
 (segment (start 23.39 40.89) (end 23.22 40.89) (width 0.25) (layer "F.Cu") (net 10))
 (segment (start 49.28 29.35) (end 59.28 29.35) (width 0.25) (layer "B.Cu") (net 13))
 (segment (start 68.525 54.875) (end 68.755 54.645) (width 0.25) (layer "B.Cu") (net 13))
 (segment (start 71.255 50.875) (end 71.255 42.755) (width 0.25) (layer "B.Cu") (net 13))
 (segment (start 65.95 51.1) (end 65.95 53.52) (width 0.25) (layer "B.Cu") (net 13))
 (segment (start 21.5 44.35) (end 21.77 44.08) (width 0.25) (layer "B.Cu") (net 13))
 (segment (start 68.755 53.755) (end 68.755 54.645) (width 0.25) (layer "B.Cu") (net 13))
 (segment (start 21.78 44.08) (end 21.78 41.85) (width 0.25) (layer "B.Cu") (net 13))
 (segment (start 21.5 44.35) (end 21.76 44.35) (width 0.25) (layer "B.Cu") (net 13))
 (segment (start 60.125 29.875) (end 60.09 29.91) (width 0.25) (layer "B.Cu") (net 13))
 (segment (start 21.515 26.585) (end 21.595 26.665) (width 0.25) (layer "B.Cu") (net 13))
 (segment (start 63.28 33.35) (end 63.28 35.35) (width 0.25) (layer "B.Cu") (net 13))
 (segment (start 22.3 46.85) (end 22.1 46.85) (width 0.25) (layer "B.Cu") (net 13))
 (segment (start 21.78 41.85) (end 21.78 44.37) (width 0.25) (layer "B.Cu") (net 13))
 (segment (start 71.255 50.875) (end 71.03 51.1) (width 0.25) (layer "B.Cu") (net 13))
 (segment (start 65.95 53.52) (end 67.305 54.875) (width 0.25) (layer "B.Cu") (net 13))
 (segment (start 72.53 51.1) (end 71.03 51.1) (width 0.25) (layer "B.Cu") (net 13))
 (segment (start 21.77 44.08) (end 21.78 44.08) (width 0.25) (layer "B.Cu") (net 13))
 (segment (start 18.68 24.35) (end 19.28 24.35) (width 0.25) (layer "B.Cu") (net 13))
 (segment (start 71.255 32.495) (end 74.55 29.2) (width 0.25) (layer "B.Cu") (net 13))
 (segment (start 65.45 29.2) (end 60.8 29.2) (width 0.25) (layer "B.Cu") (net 13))
 (segment (start 71.255 50.875) (end 71.48 51.1) (width 0.25) (layer "B.Cu") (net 13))
 (segment (start 71.48 51.1) (end 72.53 51.1) (width 0.25) (layer "B.Cu") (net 13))
 (segment (start 19.28 24.35) (end 21.515 26.585) (width 0.25) (layer "B.Cu") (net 13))
 (segment (start 67.5 57.5) (end 68.755 56.245) (width 0.25) (layer "B.Cu") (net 13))
 (segment (start 67.305 54.875) (end 68.525 54.875) (width 0.25) (layer "B.Cu") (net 13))
 (segment (start 71.03 51.1) (end 70.03 51.1) (width 0.25) (layer "B.Cu") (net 13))
 (segment (start 62.715 32.785) (end 62.68 32.75) (width 0.25) (layer "B.Cu") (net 13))
 (segment (start 45.52 21.875) (end 45.52 25.59) (width 0.25) (layer "B.Cu") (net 13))
 (segment (start 22.05 46.85) (end 21.78 46.58) (width 0.25) (layer "B.Cu") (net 13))
 (segment (start 21.965 26.665) (end 21.78 26.85) (width 0.25) (layer "B.Cu") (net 13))
 (segment (start 22.5 57.5) (end 67.5 57.5) (width 0.25) (layer "B.Cu") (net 13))
 (segment (start 68.755 55.055) (end 68.755 53.755) (width 0.25) (layer "B.Cu") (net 13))
 (segment (start 71.255 42.245) (end 71.255 32.495) (width 0.25) (layer "B.Cu") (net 13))
 (segment (start 20.73 44.35) (end 21.5 44.35) (width 0.25) (layer "B.Cu") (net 13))
 (segment (start 62.25 32.75) (end 60 35) (width 0.25) (layer "B.Cu") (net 13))
 (segment (start 59.875 29.875) (end 60.125 29.875) (width 0.25) (layer "B.Cu") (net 13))
 (segment (start 68.525 54.875) (end 68.705 55.055) (width 0.25) (layer "B.Cu") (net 13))
 (segment (start 19.23 45.85) (end 20.73 44.35) (width 0.25) (layer "B.Cu") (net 13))
 (segment (start 71 42.5) (end 71.255 42.755) (width 0.25) (layer "B.Cu") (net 13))
 (segment (start 21.78 46.58) (end 21.78 56.78) (width 0.25) (layer "B.Cu") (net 13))
 (segment (start 70.03 51.1) (end 68.755 52.375) (width 0.25) (layer "B.Cu") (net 13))
 (segment (start 21.78 44.37) (end 21.78 46.58) (width 0.25) (layer "B.Cu") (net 13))
 (segment (start 60.09 30.16) (end 62.465 32.535) (width 0.25) (layer "B.Cu") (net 13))
 (segment (start 60.09 29.91) (end 60.09 30.16) (width 0.25) (layer "B.Cu") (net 13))
 (segment (start 27.78 24.35) (end 24.28 24.35) (width 0.25) (layer "B.Cu") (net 13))
 (segment (start 75.05 51.1) (end 72.53 51.1) (width 0.25) (layer "B.Cu") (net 13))
 (segment (start 71.255 42.755) (end 71.255 42.245) (width 0.25) (layer "B.Cu") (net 13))
 (segment (start 60.8 29.2) (end 60.125 29.875) (width 0.25) (layer "B.Cu") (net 13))
 (segment (start 60.125 29.875) (end 59.965 30.035) (width 0.25) (layer "B.Cu") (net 13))
 (segment (start 21.76 44.35) (end 21.78 44.37) (width 0.25) (layer "B.Cu") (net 13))
 (segment (start 59.84 29.91) (end 59.965 30.035) (width 0.25) (layer "B.Cu") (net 13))
 (segment (start 24.28 24.35) (end 21.965 26.665) (width 0.25) (layer "B.Cu") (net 13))
 (segment (start 68.705 55.055) (end 68.755 55.055) (width 0.25) (layer "B.Cu") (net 13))
 (segment (start 45.52 25.59) (end 49.28 29.35) (width 0.25) (layer "B.Cu") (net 13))
 (segment (start 60 42.5) (end 62.5 45) (width 0.25) (layer "B.Cu") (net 13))
 (segment (start 28.33 45.85) (end 27.33 46.85) (width 0.25) (layer "B.Cu") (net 13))
 (segment (start 68.755 56.245) (end 68.755 55.055) (width 0.25) (layer "B.Cu") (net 13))
 (segment (start 21.78 56.78) (end 22.5 57.5) (width 0.25) (layer "B.Cu") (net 13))
 (segment (start 21.595 26.665) (end 21.965 26.665) (width 0.25) (layer "B.Cu") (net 13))
 (segment (start 62.715 32.785) (end 63.28 33.35) (width 0.25) (layer "B.Cu") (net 13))
 (segment (start 59.28 29.35) (end 59.84 29.91) (width 0.25) (layer "B.Cu") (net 13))
 (segment (start 59.84 29.91) (end 59.875 29.875) (width 0.25) (layer "B.Cu") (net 13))
 (segment (start 68.755 52.375) (end 68.755 53.755) (width 0.25) (layer "B.Cu") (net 13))
 (segment (start 67.5 42.5) (end 71 42.5) (width 0.25) (layer "B.Cu") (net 13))
 (segment (start 65 45) (end 67.5 42.5) (width 0.25) (layer "B.Cu") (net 13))
 (segment (start 22.3 46.85) (end 22.05 46.85) (width 0.25) (layer "B.Cu") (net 13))
 (segment (start 27.33 46.85) (end 22.3 46.85) (width 0.25) (layer "B.Cu") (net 13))
 (segment (start 60 35) (end 60 42.5) (width 0.25) (layer "B.Cu") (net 13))
 (segment (start 59.965 30.035) (end 60.09 30.16) (width 0.25) (layer "B.Cu") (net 13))
 (segment (start 21.515 26.585) (end 21.78 26.85) (width 0.25) (layer "B.Cu") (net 13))
 (segment (start 21.78 26.85) (end 21.78 41.85) (width 0.25) (layer "B.Cu") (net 13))
 (segment (start 62.465 32.535) (end 62.715 32.785) (width 0.25) (layer "B.Cu") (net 13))
 (segment (start 62.68 32.75) (end 62.25 32.75) (width 0.25) (layer "B.Cu") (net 13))
 (segment (start 71 42.5) (end 71.255 42.245) (width 0.25) (layer "B.Cu") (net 13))
 (segment (start 62.465 32.535) (end 62.25 32.75) (width 0.25) (layer "B.Cu") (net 13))
 (segment (start 22.1 46.85) (end 21.78 47.17) (width 0.25) (layer "B.Cu") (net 13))
 (segment (start 62.5 45) (end 65 45) (width 0.25) (layer "B.Cu") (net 13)))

